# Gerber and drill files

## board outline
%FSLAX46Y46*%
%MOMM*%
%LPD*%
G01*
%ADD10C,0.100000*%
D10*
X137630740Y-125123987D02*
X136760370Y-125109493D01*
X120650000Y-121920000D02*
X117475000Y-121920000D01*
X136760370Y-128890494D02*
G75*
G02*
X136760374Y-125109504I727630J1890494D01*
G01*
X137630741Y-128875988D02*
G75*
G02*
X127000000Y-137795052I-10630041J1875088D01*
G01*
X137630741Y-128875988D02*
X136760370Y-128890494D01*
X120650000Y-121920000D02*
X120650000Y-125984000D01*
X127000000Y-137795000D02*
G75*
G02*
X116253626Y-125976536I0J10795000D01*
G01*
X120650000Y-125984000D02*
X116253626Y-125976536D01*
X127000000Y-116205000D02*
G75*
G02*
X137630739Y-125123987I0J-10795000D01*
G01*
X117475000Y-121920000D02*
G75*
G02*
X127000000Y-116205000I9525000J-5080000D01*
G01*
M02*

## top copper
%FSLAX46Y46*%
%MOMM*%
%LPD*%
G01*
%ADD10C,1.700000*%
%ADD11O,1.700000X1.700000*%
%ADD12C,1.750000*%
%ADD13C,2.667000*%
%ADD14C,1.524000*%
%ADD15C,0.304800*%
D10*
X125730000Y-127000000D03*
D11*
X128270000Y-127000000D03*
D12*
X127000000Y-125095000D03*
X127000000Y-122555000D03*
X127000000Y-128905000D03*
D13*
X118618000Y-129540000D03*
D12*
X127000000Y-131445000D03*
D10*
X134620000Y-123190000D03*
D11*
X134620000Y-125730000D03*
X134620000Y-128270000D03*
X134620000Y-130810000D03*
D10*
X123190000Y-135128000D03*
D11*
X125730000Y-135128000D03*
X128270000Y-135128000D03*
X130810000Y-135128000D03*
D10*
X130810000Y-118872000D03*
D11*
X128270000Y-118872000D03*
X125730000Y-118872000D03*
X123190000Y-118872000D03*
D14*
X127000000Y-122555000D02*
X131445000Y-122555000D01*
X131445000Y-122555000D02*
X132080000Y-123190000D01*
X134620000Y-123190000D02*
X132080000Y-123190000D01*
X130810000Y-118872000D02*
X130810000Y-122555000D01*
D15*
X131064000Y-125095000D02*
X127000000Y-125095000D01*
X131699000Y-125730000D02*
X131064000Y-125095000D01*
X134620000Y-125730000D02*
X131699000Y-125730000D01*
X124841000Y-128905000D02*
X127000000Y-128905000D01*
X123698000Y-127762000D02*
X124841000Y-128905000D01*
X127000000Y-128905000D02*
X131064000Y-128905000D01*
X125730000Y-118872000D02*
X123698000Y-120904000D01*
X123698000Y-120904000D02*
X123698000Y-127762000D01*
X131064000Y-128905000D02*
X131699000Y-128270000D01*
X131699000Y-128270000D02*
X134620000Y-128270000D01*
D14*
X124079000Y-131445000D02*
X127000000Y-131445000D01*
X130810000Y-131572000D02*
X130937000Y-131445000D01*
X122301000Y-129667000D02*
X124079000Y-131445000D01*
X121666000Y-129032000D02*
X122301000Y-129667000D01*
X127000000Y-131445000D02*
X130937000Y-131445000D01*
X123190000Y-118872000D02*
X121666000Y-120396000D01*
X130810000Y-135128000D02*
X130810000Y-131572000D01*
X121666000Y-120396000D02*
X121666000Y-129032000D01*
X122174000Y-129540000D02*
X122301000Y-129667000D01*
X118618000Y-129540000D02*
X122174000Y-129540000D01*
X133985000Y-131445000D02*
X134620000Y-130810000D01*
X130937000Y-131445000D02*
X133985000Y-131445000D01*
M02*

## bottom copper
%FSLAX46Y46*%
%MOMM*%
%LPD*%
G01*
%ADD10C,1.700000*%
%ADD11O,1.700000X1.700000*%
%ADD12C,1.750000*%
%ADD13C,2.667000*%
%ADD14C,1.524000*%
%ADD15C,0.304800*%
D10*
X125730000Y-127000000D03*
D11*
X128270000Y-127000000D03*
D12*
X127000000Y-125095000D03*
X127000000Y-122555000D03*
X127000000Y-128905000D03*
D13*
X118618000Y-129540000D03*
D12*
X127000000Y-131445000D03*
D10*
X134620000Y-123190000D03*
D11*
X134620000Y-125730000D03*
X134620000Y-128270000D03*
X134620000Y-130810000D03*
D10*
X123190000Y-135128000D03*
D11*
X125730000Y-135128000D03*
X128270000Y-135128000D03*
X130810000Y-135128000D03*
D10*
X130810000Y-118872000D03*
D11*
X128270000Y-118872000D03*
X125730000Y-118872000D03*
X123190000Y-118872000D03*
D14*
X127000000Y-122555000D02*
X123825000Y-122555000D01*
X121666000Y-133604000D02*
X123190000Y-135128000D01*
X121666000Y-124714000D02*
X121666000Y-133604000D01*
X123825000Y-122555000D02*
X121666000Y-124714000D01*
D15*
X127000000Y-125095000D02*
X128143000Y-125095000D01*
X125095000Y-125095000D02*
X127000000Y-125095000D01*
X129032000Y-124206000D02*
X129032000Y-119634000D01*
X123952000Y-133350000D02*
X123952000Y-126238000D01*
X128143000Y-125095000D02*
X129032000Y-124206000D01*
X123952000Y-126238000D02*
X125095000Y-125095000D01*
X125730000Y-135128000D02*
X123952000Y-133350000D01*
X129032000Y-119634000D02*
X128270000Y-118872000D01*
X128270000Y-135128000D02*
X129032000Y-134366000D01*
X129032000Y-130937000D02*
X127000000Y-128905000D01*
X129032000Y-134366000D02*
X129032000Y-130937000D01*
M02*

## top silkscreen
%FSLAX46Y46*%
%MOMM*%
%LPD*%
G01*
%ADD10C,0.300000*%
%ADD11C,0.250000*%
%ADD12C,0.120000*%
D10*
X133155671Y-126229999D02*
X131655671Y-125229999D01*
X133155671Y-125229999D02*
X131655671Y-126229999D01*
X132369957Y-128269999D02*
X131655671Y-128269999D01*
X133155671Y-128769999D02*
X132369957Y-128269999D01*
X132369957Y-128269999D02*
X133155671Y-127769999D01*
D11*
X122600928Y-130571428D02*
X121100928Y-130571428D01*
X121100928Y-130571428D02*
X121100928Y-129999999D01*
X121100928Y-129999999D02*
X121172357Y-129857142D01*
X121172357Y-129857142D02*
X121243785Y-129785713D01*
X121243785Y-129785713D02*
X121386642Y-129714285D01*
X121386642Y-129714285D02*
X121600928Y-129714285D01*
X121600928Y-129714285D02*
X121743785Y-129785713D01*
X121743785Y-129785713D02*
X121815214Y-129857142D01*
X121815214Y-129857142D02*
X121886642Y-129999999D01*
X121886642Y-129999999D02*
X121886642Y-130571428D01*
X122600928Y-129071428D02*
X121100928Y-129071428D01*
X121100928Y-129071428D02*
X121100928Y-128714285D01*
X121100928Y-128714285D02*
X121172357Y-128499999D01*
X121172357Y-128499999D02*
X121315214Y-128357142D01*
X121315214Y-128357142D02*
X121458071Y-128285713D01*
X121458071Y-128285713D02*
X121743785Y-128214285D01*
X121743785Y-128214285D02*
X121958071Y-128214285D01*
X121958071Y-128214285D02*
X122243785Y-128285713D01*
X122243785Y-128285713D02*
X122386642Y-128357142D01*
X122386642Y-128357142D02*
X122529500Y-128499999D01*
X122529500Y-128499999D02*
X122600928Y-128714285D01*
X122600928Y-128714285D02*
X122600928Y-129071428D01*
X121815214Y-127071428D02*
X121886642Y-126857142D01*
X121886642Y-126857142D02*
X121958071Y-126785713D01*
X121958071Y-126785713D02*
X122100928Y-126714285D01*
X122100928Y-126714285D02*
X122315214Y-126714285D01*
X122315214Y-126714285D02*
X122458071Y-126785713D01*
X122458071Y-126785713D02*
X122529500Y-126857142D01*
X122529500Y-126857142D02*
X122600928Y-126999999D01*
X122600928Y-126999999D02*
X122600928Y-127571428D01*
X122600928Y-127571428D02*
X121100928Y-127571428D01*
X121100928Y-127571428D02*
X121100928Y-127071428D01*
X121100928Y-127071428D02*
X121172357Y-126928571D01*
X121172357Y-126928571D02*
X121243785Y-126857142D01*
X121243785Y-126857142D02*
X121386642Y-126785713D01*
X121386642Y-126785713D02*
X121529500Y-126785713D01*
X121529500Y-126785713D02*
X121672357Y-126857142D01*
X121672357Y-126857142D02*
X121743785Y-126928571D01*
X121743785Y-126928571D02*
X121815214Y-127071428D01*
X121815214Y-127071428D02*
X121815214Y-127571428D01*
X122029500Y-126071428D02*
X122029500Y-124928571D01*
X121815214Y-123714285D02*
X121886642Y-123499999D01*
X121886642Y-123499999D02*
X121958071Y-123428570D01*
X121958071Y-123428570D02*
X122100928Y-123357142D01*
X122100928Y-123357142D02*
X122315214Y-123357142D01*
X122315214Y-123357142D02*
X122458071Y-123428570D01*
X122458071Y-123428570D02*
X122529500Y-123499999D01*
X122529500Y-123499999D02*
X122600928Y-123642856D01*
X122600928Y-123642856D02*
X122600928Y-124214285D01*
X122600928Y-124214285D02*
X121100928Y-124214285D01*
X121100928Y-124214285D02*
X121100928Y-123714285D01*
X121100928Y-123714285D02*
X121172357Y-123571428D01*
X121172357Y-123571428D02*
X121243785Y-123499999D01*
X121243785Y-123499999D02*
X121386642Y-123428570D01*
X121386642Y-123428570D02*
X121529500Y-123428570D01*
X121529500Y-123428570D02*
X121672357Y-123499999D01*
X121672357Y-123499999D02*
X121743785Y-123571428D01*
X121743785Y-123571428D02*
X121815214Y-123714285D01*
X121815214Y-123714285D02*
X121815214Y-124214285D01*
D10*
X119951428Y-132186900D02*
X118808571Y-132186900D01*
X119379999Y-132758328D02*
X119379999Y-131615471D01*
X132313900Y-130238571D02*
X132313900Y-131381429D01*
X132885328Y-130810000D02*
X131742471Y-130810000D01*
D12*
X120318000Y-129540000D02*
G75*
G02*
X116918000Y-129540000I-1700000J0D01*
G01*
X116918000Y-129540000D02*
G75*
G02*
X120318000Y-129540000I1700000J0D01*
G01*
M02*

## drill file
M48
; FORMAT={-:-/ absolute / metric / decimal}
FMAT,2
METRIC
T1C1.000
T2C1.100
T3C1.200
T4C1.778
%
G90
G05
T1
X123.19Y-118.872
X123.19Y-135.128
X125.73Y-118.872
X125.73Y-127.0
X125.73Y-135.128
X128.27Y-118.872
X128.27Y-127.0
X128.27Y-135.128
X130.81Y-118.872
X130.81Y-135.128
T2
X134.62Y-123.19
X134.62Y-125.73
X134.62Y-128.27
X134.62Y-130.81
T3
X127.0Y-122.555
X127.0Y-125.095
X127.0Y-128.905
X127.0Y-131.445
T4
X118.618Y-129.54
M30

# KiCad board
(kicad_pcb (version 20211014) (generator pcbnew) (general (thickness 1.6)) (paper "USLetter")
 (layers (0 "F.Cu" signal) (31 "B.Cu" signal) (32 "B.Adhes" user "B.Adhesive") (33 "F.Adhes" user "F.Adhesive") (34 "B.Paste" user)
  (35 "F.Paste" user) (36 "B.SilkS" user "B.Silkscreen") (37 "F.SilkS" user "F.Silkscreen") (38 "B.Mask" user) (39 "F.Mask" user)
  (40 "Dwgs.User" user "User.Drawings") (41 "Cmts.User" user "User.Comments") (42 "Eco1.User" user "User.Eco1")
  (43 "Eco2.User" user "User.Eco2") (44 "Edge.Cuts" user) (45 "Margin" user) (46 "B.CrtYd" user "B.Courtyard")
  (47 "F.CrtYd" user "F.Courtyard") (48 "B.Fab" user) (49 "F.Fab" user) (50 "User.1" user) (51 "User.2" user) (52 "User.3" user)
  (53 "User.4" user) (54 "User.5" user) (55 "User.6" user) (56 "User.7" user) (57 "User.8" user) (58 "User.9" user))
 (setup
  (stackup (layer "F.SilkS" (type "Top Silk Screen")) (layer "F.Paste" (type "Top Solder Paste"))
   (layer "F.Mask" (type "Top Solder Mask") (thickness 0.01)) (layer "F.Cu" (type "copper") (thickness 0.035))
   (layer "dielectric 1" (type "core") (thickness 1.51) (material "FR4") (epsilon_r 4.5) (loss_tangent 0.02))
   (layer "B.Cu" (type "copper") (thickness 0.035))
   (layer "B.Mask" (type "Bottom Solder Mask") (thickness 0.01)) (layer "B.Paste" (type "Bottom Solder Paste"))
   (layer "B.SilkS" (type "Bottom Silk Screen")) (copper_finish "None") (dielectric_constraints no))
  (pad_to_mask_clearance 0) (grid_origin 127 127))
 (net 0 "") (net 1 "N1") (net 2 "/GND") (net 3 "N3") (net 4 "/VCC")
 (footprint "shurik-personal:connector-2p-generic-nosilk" (layer "F.Cu") (at 125.73 127 90)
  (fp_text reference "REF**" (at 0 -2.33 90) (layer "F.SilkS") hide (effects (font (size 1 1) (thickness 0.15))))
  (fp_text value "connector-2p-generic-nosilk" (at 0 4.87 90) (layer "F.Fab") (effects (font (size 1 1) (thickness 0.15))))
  (pad "1" thru_hole circle (at 0 0 90) (size 1.7 1.7) (drill 1) (layers *.Cu *.Mask))
  (pad "2" thru_hole oval (at 0 2.54 90) (size 1.7 1.7) (drill 1) (layers *.Cu *.Mask)))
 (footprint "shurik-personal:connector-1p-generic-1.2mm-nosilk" (layer "F.Cu") (at 127 125.095)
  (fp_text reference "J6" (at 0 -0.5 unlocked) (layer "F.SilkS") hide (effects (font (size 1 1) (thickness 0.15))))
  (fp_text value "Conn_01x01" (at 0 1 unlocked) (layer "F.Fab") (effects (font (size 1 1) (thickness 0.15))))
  (pad "1" thru_hole circle (at 0 0) (size 1.75 1.75) (drill 1.2) (layers *.Cu *.Mask) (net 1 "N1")))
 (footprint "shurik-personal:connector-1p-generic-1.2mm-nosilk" (layer "F.Cu") (at 127 122.555)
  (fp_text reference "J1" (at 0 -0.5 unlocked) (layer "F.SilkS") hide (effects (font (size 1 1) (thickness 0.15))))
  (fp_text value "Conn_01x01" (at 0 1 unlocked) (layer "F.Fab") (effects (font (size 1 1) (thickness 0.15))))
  (pad "1" thru_hole circle (at 0 0) (size 1.75 1.75) (drill 1.2) (layers *.Cu *.Mask) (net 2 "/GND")))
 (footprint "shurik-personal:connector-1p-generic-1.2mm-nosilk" (layer "F.Cu") (at 127 128.905)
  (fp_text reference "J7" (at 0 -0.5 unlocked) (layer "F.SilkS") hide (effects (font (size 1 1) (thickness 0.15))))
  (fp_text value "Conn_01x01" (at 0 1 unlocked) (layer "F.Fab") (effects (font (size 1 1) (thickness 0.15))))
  (pad "1" thru_hole circle (at 0 0) (size 1.75 1.75) (drill 1.2) (layers *.Cu *.Mask) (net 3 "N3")))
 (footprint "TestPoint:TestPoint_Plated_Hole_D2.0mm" (layer "F.Cu") (at 118.618 129.54)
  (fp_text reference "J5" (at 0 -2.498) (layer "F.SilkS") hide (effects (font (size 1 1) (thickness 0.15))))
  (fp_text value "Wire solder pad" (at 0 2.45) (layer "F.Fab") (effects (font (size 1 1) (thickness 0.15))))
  (fp_circle (center 0 0) (end 0 -1.7) (layer "F.SilkS") (width 0.12) (fill none))
  (pad "1" thru_hole circle (at 0 0) (size 2.667 2.667) (drill 1.778) (layers *.Cu *.Mask) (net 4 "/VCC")))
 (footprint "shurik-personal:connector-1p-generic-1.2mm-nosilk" (layer "F.Cu") (at 127 131.445)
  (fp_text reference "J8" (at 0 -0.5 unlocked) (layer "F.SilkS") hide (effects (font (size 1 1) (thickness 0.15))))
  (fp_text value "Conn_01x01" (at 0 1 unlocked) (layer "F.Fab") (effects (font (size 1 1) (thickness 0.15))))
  (pad "1" thru_hole circle (at 0 0) (size 1.75 1.75) (drill 1.2) (layers *.Cu *.Mask) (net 4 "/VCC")))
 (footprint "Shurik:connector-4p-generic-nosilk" (layer "F.Cu") (at 134.62 123.19)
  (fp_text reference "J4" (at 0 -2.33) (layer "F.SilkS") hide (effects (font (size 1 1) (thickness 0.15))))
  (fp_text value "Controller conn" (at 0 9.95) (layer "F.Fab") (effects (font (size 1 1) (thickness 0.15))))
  (pad "1" thru_hole circle (at 0 0) (size 1.7 1.7) (drill 1.1) (layers *.Cu *.Mask) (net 2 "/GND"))
  (pad "2" thru_hole oval (at 0 2.54) (size 1.7 1.7) (drill 1.1) (layers *.Cu *.Mask) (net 1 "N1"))
  (pad "3" thru_hole oval (at 0 5.08) (size 1.7 1.7) (drill 1.1) (layers *.Cu *.Mask) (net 3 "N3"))
  (pad "4" thru_hole oval (at 0 7.62) (size 1.7 1.7) (drill 1.1) (layers *.Cu *.Mask) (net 4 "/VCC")))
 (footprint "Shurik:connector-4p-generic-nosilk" (layer "F.Cu") (at 123.19 135.128 90)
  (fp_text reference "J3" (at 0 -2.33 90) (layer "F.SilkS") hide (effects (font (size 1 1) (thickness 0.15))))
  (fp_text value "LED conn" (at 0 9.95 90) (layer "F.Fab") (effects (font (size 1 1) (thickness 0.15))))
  (pad "1" thru_hole circle (at 0 0 90) (size 1.7 1.7) (drill 1) (layers *.Cu *.Mask) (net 2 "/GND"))
  (pad "2" thru_hole oval (at 0 2.54 90) (size 1.7 1.7) (drill 1) (layers *.Cu *.Mask) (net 1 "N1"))
  (pad "3" thru_hole oval (at 0 5.08 90) (size 1.7 1.7) (drill 1) (layers *.Cu *.Mask) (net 3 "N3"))
  (pad "4" thru_hole oval (at 0 7.62 90) (size 1.7 1.7) (drill 1) (layers *.Cu *.Mask) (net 4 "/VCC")))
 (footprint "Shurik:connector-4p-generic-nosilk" (layer "F.Cu") (at 130.81 118.872 -90)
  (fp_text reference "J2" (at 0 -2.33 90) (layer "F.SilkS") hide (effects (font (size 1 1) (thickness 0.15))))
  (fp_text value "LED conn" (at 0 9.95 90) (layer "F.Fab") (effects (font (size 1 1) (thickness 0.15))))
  (pad "1" thru_hole circle (at 0 0 270) (size 1.7 1.7) (drill 1) (layers *.Cu *.Mask) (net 2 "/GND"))
  (pad "2" thru_hole oval (at 0 2.54 270) (size 1.7 1.7) (drill 1) (layers *.Cu *.Mask) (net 1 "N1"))
  (pad "3" thru_hole oval (at 0 5.08 270) (size 1.7 1.7) (drill 1) (layers *.Cu *.Mask) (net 3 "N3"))
  (pad "4" thru_hole oval (at 0 7.62 270) (size 1.7 1.7) (drill 1) (layers *.Cu *.Mask) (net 4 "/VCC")))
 (gr_line (start 137.63074 125.123987) (end 136.76037 125.109493) (layer "Edge.Cuts") (width 0.1))
 (gr_line (start 120.65 121.92) (end 117.475 121.92) (layer "Edge.Cuts") (width 0.1))
 (gr_arc (start 136.76037 128.890494) (mid 135.462276 126.999993) (end 136.76037 125.109493) (layer "Edge.Cuts") (width 0.1))
 (gr_arc (start 137.630741 128.875988) (mid 133.938498 135.27013) (end 127 137.795) (layer "Edge.Cuts") (width 0.1))
 (gr_line (start 137.630741 128.875988) (end 136.76037 128.890494) (layer "Edge.Cuts") (width 0.1))
 (gr_line (start 120.65 121.92) (end 120.65 125.984) (layer "Edge.Cuts") (width 0.1))
 (gr_arc (start 127 137.795) (mid 119.013129 134.262356) (end 116.253626 125.976536) (layer "Edge.Cuts") (width 0.1))
 (gr_line (start 120.65 125.984) (end 116.253626 125.976536) (layer "Edge.Cuts") (width 0.1))
 (gr_arc (start 127 116.205) (mid 133.93832 118.730063) (end 137.63074 125.123987) (layer "Edge.Cuts") (width 0.1))
 (gr_arc (start 117.475 121.92) (mid 121.446017 117.743361) (end 127 116.205) (layer "Edge.Cuts") (width 0.1))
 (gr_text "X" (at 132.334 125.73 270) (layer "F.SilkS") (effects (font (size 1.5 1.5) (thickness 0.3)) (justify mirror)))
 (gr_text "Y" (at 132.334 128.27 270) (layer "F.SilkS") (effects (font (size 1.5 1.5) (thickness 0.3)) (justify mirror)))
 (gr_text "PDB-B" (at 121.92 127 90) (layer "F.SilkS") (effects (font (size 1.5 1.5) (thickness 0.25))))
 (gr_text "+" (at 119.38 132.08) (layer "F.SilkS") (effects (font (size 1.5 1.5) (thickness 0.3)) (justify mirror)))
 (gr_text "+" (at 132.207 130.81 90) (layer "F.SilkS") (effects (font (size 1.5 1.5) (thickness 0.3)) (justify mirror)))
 (segment (start 127 122.555) (end 131.445 122.555) (width 1.524) (layer "F.Cu") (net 2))
 (segment (start 131.445 122.555) (end 132.08 123.19) (width 1.524) (layer "F.Cu") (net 2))
 (segment (start 134.62 123.19) (end 132.08 123.19) (width 1.524) (layer "F.Cu") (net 2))
 (segment (start 130.81 118.872) (end 130.81 122.555) (width 1.524) (layer "F.Cu") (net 2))
 (segment (start 127 122.555) (end 123.825 122.555) (width 1.524) (layer "B.Cu") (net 2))
 (segment (start 121.666 133.604) (end 123.19 135.128) (width 1.524) (layer "B.Cu") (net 2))
 (segment (start 121.666 124.714) (end 121.666 133.604) (width 1.524) (layer "B.Cu") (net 2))
 (segment (start 123.825 122.555) (end 121.666 124.714) (width 1.524) (layer "B.Cu") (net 2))
 (segment (start 131.064 125.095) (end 127 125.095) (width 0.3048) (layer "F.Cu") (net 1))
 (segment (start 131.699 125.73) (end 131.064 125.095) (width 0.3048) (layer "F.Cu") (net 1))
 (segment (start 134.62 125.73) (end 131.699 125.73) (width 0.3048) (layer "F.Cu") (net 1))
 (segment (start 127 125.095) (end 128.143 125.095) (width 0.3048) (layer "B.Cu") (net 1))
 (segment (start 125.095 125.095) (end 127 125.095) (width 0.3048) (layer "B.Cu") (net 1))
 (segment (start 129.032 124.206) (end 129.032 119.634) (width 0.3048) (layer "B.Cu") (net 1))
 (segment (start 123.952 133.35) (end 123.952 126.238) (width 0.3048) (layer "B.Cu") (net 1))
 (segment (start 128.143 125.095) (end 129.032 124.206) (width 0.3048) (layer "B.Cu") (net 1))
 (segment (start 123.952 126.238) (end 125.095 125.095) (width 0.3048) (layer "B.Cu") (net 1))
 (segment (start 125.73 135.128) (end 123.952 133.35) (width 0.3048) (layer "B.Cu") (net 1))
 (segment (start 129.032 119.634) (end 128.27 118.872) (width 0.3048) (layer "B.Cu") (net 1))
 (segment (start 124.841 128.905) (end 127 128.905) (width 0.3048) (layer "F.Cu") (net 3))
 (segment (start 123.698 127.762) (end 124.841 128.905) (width 0.3048) (layer "F.Cu") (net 3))
 (segment (start 127 128.905) (end 131.064 128.905) (width 0.3048) (layer "F.Cu") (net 3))
 (segment (start 125.73 118.872) (end 123.698 120.904) (width 0.3048) (layer "F.Cu") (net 3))
 (segment (start 123.698 120.904) (end 123.698 127.762) (width 0.3048) (layer "F.Cu") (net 3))
 (segment (start 131.064 128.905) (end 131.699 128.27) (width 0.3048) (layer "F.Cu") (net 3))
 (segment (start 131.699 128.27) (end 134.62 128.27) (width 0.3048) (layer "F.Cu") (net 3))
 (segment (start 128.27 135.128) (end 129.032 134.366) (width 0.3048) (layer "B.Cu") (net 3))
 (segment (start 129.032 130.937) (end 127 128.905) (width 0.3048) (layer "B.Cu") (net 3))
 (segment (start 129.032 134.366) (end 129.032 130.937) (width 0.3048) (layer "B.Cu") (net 3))
 (segment (start 124.079 131.445) (end 127 131.445) (width 1.524) (layer "F.Cu") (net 4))
 (segment (start 130.81 131.572) (end 130.937 131.445) (width 1.524) (layer "F.Cu") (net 4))
 (segment (start 122.301 129.667) (end 124.079 131.445) (width 1.524) (layer "F.Cu") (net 4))
 (segment (start 121.666 129.032) (end 122.301 129.667) (width 1.524) (layer "F.Cu") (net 4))
 (segment (start 127 131.445) (end 130.937 131.445) (width 1.524) (layer "F.Cu") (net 4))
 (segment (start 123.19 118.872) (end 121.666 120.396) (width 1.524) (layer "F.Cu") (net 4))
 (segment (start 130.81 135.128) (end 130.81 131.572) (width 1.524) (layer "F.Cu") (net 4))
 (segment (start 121.666 120.396) (end 121.666 129.032) (width 1.524) (layer "F.Cu") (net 4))
 (segment (start 122.174 129.54) (end 122.301 129.667) (width 1.524) (layer "F.Cu") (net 4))
 (segment (start 118.618 129.54) (end 122.174 129.54) (width 1.524) (layer "F.Cu") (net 4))
 (segment (start 133.985 131.445) (end 134.62 130.81) (width 1.524) (layer "F.Cu") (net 4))
 (segment (start 130.937 131.445) (end 133.985 131.445) (width 1.524) (layer "F.Cu") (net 4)))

